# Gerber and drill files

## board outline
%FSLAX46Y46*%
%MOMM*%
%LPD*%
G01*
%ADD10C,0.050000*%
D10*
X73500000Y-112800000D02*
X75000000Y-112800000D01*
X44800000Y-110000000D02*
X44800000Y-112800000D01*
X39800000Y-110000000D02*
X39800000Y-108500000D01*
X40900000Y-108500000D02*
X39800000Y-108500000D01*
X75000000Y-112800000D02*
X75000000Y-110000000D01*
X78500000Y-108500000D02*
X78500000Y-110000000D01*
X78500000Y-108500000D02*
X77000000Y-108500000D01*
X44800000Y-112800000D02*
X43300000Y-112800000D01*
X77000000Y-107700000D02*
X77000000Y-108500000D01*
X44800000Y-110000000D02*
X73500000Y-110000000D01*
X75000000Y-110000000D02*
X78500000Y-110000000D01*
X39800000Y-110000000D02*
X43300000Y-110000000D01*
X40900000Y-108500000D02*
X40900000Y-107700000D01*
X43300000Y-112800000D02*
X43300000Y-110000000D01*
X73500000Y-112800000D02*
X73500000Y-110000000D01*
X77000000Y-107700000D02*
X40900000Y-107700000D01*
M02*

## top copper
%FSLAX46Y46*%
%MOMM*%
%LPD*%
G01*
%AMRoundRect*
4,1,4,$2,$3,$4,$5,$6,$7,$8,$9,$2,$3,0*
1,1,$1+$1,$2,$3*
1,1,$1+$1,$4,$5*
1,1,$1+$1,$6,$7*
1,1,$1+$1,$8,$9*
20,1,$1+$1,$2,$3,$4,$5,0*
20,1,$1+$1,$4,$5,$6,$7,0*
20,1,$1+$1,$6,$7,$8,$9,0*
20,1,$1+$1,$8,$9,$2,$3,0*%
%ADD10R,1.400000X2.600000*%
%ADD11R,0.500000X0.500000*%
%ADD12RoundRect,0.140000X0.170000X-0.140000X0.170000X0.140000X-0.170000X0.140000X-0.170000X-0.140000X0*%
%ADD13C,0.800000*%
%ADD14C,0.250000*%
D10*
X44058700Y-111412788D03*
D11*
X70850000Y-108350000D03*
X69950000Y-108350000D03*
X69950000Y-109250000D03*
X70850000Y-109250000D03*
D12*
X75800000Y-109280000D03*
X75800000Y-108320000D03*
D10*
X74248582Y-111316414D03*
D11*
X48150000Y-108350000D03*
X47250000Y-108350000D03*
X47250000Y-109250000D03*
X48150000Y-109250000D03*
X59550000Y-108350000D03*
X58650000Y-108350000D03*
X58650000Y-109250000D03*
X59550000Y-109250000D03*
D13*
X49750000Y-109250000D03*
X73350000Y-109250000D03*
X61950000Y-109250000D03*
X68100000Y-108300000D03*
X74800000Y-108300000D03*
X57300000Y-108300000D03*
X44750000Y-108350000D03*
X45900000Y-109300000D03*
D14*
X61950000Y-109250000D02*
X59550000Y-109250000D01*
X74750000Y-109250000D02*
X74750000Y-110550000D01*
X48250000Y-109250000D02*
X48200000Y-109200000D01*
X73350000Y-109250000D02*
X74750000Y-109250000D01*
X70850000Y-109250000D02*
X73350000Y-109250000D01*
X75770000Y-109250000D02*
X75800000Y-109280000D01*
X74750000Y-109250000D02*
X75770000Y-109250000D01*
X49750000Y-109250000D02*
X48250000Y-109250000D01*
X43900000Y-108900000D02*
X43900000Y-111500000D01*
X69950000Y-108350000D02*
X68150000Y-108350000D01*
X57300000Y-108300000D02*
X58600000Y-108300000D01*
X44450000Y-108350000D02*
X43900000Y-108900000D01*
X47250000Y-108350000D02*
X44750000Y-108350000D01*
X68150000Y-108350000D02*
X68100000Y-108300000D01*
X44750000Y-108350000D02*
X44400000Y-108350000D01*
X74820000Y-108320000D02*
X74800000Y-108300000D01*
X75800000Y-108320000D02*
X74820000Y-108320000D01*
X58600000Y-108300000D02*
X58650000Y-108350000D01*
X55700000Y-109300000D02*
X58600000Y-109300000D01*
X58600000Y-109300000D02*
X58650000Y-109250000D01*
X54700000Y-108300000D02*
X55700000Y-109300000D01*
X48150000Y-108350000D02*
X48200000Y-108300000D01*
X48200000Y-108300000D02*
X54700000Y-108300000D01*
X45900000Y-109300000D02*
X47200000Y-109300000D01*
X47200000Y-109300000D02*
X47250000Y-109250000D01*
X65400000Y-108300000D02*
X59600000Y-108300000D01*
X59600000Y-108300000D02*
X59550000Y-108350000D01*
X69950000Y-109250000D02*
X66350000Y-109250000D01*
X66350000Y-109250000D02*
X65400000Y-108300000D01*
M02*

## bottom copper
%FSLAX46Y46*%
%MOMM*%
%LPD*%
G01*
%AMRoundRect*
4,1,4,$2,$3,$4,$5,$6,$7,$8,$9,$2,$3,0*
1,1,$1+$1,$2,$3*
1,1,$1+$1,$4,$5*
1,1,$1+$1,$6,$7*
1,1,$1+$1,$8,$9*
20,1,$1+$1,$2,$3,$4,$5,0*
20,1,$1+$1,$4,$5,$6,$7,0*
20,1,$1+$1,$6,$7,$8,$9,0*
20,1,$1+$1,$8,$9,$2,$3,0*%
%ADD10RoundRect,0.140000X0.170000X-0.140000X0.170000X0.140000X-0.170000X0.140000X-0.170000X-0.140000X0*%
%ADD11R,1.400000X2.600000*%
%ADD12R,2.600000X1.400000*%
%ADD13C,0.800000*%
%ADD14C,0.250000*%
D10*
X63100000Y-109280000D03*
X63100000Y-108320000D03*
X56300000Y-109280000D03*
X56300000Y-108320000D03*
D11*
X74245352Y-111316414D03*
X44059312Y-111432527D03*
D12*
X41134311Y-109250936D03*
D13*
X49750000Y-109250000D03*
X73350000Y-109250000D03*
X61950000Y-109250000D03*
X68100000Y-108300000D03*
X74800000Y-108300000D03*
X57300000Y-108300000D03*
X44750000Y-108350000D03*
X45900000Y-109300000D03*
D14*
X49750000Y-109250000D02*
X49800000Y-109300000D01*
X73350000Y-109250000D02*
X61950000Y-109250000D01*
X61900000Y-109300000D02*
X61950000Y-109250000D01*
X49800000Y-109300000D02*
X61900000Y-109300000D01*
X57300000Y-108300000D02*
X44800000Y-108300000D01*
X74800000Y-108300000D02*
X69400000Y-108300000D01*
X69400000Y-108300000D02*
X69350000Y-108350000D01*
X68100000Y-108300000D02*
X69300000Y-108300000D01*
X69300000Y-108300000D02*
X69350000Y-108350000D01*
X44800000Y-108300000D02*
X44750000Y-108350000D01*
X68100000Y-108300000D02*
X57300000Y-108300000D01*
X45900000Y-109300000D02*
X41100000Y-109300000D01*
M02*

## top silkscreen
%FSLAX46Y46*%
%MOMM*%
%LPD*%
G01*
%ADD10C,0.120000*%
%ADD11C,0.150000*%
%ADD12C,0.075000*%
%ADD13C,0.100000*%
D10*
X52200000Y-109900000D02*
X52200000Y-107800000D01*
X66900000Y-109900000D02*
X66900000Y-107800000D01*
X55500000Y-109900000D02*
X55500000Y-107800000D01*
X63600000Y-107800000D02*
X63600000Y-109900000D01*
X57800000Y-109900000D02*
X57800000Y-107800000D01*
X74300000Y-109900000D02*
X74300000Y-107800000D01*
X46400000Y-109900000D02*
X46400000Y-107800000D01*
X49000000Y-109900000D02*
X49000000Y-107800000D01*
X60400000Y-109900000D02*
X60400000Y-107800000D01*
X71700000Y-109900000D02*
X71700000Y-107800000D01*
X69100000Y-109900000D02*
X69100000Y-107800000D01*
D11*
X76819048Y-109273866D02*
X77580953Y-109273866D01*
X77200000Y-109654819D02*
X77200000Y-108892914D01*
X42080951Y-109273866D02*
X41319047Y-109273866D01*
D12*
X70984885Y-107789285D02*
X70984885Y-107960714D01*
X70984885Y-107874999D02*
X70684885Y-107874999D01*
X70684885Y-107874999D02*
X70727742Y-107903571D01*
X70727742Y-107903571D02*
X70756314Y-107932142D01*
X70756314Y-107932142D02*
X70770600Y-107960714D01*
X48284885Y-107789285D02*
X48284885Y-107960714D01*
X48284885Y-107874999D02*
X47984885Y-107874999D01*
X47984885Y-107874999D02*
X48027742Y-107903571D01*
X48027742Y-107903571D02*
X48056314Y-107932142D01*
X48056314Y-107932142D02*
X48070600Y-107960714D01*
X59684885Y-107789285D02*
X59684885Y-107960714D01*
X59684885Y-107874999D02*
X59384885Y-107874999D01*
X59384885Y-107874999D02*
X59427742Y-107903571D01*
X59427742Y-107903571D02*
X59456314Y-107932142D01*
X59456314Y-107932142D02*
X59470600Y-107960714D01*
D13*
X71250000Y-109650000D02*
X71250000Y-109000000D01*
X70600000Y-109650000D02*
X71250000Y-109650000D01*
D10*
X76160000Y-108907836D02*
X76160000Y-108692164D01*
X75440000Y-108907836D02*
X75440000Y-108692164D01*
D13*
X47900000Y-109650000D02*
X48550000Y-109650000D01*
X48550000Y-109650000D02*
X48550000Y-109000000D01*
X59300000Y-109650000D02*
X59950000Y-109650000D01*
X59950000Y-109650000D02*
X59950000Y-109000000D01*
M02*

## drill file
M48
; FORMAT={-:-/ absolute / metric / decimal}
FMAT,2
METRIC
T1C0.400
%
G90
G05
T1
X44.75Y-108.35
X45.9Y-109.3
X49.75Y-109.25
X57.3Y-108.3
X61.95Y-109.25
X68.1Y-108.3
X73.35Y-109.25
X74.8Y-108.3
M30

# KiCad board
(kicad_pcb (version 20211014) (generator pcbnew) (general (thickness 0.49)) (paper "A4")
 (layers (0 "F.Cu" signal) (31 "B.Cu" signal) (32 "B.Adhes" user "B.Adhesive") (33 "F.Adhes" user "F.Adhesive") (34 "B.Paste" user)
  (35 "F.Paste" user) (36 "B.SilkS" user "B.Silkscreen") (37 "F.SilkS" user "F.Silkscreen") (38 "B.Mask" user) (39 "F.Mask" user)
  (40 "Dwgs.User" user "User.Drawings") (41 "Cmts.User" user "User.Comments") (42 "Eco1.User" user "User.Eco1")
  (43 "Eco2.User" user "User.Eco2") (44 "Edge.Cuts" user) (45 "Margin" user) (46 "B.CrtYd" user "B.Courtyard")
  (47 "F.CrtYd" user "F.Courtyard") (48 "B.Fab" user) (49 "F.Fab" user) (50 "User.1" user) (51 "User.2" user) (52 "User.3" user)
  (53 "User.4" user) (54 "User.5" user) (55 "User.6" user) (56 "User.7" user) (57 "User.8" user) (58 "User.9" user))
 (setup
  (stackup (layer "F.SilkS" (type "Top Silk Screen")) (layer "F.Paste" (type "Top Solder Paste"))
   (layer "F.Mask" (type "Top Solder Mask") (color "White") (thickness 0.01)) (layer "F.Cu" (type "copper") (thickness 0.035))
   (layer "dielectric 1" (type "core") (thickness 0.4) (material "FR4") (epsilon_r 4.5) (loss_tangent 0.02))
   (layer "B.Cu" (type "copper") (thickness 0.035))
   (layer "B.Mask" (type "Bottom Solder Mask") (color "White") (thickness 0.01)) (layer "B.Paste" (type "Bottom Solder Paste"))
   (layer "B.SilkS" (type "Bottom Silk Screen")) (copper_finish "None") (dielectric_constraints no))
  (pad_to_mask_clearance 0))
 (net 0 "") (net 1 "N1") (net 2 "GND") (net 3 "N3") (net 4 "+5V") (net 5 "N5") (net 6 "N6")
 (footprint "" (layer "F.Cu") (at 44.0587 111.412788)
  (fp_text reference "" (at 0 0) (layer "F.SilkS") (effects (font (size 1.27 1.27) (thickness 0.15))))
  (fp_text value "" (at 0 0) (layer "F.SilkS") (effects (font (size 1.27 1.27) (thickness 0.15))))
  (pad "" smd rect (at 0 0) (size 1.4 2.6) (layers "F.Cu" "F.Paste" "F.Mask")))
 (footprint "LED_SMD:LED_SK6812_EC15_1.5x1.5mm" (layer "F.Cu") (at 70.4 108.8 -90)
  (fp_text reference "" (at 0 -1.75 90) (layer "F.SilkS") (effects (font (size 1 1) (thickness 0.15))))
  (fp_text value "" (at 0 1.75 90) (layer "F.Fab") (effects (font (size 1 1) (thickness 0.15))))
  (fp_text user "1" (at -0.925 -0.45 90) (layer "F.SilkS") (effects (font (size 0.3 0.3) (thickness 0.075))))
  (fp_line (start 0.85 -0.85) (end 0.2 -0.85) (layer "F.SilkS") (width 0.1))
  (fp_line (start 0.85 -0.2) (end 0.85 -0.85) (layer "F.SilkS") (width 0.1))
  (pad "1" smd rect (at -0.45 -0.45 270) (size 0.5 0.5) (layers "F.Cu" "F.Paste" "F.Mask") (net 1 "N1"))
  (pad "2" smd rect (at -0.45 0.45 270) (size 0.5 0.5) (layers "F.Cu" "F.Paste" "F.Mask") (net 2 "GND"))
  (pad "3" smd rect (at 0.45 0.45 270) (size 0.5 0.5) (layers "F.Cu" "F.Paste" "F.Mask") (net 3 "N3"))
  (pad "4" smd rect (at 0.45 -0.45 270) (size 0.5 0.5) (layers "F.Cu" "F.Paste" "F.Mask") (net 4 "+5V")))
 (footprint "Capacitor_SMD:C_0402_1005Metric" (layer "F.Cu") (at 75.8 108.8 90)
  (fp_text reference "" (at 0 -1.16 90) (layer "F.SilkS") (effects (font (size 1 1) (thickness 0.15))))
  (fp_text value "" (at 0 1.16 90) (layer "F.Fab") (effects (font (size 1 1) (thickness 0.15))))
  (fp_line (start -0.107836 0.36) (end 0.107836 0.36) (layer "F.SilkS") (width 0.12))
  (fp_line (start -0.107836 -0.36) (end 0.107836 -0.36) (layer "F.SilkS") (width 0.12))
  (pad "1" smd roundrect (at -0.48 0 90) (size 0.56 0.62) (layers "F.Cu" "F.Paste" "F.Mask") (roundrect_rratio 0.25) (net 4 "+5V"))
  (pad "2" smd roundrect (at 0.48 0 90) (size 0.56 0.62) (layers "F.Cu" "F.Paste" "F.Mask") (roundrect_rratio 0.25) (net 2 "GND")))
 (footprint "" (layer "F.Cu") (at 74.248582 111.316414)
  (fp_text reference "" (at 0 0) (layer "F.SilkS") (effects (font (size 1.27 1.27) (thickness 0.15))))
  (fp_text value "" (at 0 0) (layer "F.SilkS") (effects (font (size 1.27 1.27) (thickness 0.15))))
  (pad "" smd rect (at 0 0) (size 1.4 2.6) (layers "F.Cu" "F.Paste" "F.Mask")))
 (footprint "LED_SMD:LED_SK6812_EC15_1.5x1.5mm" (layer "F.Cu") (at 47.7 108.8 -90)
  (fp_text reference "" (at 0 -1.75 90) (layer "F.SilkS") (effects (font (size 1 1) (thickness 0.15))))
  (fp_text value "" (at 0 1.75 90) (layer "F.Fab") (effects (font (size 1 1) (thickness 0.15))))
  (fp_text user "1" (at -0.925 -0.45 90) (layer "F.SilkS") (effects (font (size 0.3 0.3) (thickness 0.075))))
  (fp_line (start 0.85 -0.2) (end 0.85 -0.85) (layer "F.SilkS") (width 0.1))
  (fp_line (start 0.85 -0.85) (end 0.2 -0.85) (layer "F.SilkS") (width 0.1))
  (pad "1" smd rect (at -0.45 -0.45 270) (size 0.5 0.5) (layers "F.Cu" "F.Paste" "F.Mask") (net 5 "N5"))
  (pad "2" smd rect (at -0.45 0.45 270) (size 0.5 0.5) (layers "F.Cu" "F.Paste" "F.Mask") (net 2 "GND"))
  (pad "3" smd rect (at 0.45 0.45 270) (size 0.5 0.5) (layers "F.Cu" "F.Paste" "F.Mask") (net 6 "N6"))
  (pad "4" smd rect (at 0.45 -0.45 270) (size 0.5 0.5) (layers "F.Cu" "F.Paste" "F.Mask") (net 4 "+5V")))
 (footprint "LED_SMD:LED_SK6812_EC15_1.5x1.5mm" (layer "F.Cu") (at 59.1 108.8 -90)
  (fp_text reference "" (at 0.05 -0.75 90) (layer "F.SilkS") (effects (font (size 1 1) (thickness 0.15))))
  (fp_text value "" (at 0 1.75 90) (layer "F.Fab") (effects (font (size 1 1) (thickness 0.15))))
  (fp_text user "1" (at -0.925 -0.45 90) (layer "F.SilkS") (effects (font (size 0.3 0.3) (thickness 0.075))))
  (fp_line (start 0.85 -0.2) (end 0.85 -0.85) (layer "F.SilkS") (width 0.1))
  (fp_line (start 0.85 -0.85) (end 0.2 -0.85) (layer "F.SilkS") (width 0.1))
  (pad "1" smd rect (at -0.45 -0.45 270) (size 0.5 0.5) (layers "F.Cu" "F.Paste" "F.Mask") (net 3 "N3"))
  (pad "2" smd rect (at -0.45 0.45 270) (size 0.5 0.5) (layers "F.Cu" "F.Paste" "F.Mask") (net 2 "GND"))
  (pad "3" smd rect (at 0.45 0.45 270) (size 0.5 0.5) (layers "F.Cu" "F.Paste" "F.Mask") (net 5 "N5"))
  (pad "4" smd rect (at 0.45 -0.45 270) (size 0.5 0.5) (layers "F.Cu" "F.Paste" "F.Mask") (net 4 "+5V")))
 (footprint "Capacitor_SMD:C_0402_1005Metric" (layer "B.Cu") (at 63.1 108.8 90)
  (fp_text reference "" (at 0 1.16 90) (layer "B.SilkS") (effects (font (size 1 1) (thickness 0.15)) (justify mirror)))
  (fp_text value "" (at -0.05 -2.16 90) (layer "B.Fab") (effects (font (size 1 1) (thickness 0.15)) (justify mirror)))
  (pad "1" smd roundrect (at -0.48 0 90) (size 0.56 0.62) (layers "B.Cu" "B.Paste" "B.Mask") (roundrect_rratio 0.25))
  (pad "2" smd roundrect (at 0.48 0 90) (size 0.56 0.62) (layers "B.Cu" "B.Paste" "B.Mask") (roundrect_rratio 0.25)))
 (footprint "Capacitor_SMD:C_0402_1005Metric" (layer "B.Cu") (at 56.3 108.8 90)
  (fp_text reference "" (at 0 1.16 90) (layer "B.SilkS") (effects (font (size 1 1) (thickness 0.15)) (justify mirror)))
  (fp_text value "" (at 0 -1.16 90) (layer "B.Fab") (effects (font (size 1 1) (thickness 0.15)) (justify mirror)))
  (pad "1" smd roundrect (at -0.48 0 90) (size 0.56 0.62) (layers "B.Cu" "B.Paste" "B.Mask") (roundrect_rratio 0.25))
  (pad "2" smd roundrect (at 0.48 0 90) (size 0.56 0.62) (layers "B.Cu" "B.Paste" "B.Mask") (roundrect_rratio 0.25)))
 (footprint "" (layer "B.Cu") (at 74.245352 111.316414 180)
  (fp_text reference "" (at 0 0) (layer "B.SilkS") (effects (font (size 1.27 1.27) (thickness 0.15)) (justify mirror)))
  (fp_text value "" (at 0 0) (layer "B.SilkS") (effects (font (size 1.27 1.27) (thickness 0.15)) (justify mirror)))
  (pad "" smd rect (at 0 0 180) (size 1.4 2.6) (layers "B.Cu" "B.Paste" "B.Mask")))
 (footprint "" (layer "B.Cu") (at 44.059312 111.432527 180)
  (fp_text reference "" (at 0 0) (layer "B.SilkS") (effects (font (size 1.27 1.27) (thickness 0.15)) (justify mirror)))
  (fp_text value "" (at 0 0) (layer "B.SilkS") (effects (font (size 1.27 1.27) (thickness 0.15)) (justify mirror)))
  (pad "" smd rect (at 0 0 180) (size 1.4 2.6) (layers "B.Cu" "B.Paste" "B.Mask")))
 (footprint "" (layer "B.Cu") (at 41.134311 109.250936 90)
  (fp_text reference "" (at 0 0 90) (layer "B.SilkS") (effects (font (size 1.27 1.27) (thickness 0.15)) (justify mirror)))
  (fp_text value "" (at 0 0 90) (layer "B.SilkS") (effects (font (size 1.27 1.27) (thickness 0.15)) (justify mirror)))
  (pad "" smd rect (at 0 0 90) (size 1.4 2.6) (layers "B.Cu" "B.Paste" "B.Mask")))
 (gr_line (start 52.2 109.9) (end 52.2 107.8) (layer "F.SilkS") (width 0.12))
 (gr_line (start 66.9 109.9) (end 66.9 107.8) (layer "F.SilkS") (width 0.12))
 (gr_line (start 55.5 109.9) (end 55.5 107.8) (layer "F.SilkS") (width 0.12))
 (gr_line (start 63.6 107.8) (end 63.6 109.9) (layer "F.SilkS") (width 0.12))
 (gr_line (start 57.8 109.9) (end 57.8 107.8) (layer "F.SilkS") (width 0.12))
 (gr_line (start 74.3 109.9) (end 74.3 107.8) (layer "F.SilkS") (width 0.12))
 (gr_line (start 46.4 109.9) (end 46.4 107.8) (layer "F.SilkS") (width 0.12))
 (gr_line (start 49 109.9) (end 49 107.8) (layer "F.SilkS") (width 0.12))
 (gr_line (start 60.4 109.9) (end 60.4 107.8) (layer "F.SilkS") (width 0.12))
 (gr_line (start 71.7 109.9) (end 71.7 107.8) (layer "F.SilkS") (width 0.12))
 (gr_line (start 69.1 109.9) (end 69.1 107.8) (layer "F.SilkS") (width 0.12))
 (gr_line (start 73.5 112.8) (end 75 112.8) (layer "Edge.Cuts") (width 0.05))
 (gr_line (start 44.8 110) (end 44.8 112.8) (layer "Edge.Cuts") (width 0.05))
 (gr_line (start 39.8 110) (end 39.8 108.5) (layer "Edge.Cuts") (width 0.05))
 (gr_line (start 40.9 108.5) (end 39.8 108.5) (layer "Edge.Cuts") (width 0.05))
 (gr_line (start 75 112.8) (end 75 110) (layer "Edge.Cuts") (width 0.05))
 (gr_line (start 78.5 108.5) (end 78.5 110) (layer "Edge.Cuts") (width 0.05))
 (gr_line (start 78.5 108.5) (end 77 108.5) (layer "Edge.Cuts") (width 0.05))
 (gr_line (start 44.8 112.8) (end 43.3 112.8) (layer "Edge.Cuts") (width 0.05))
 (gr_line (start 77 107.7) (end 77 108.5) (layer "Edge.Cuts") (width 0.05))
 (gr_line (start 44.8 110) (end 73.5 110) (layer "Edge.Cuts") (width 0.05))
 (gr_line (start 75 110) (end 78.5 110) (layer "Edge.Cuts") (width 0.05))
 (gr_line (start 39.8 110) (end 43.3 110) (layer "Edge.Cuts") (width 0.05))
 (gr_line (start 40.9 108.5) (end 40.9 107.7) (layer "Edge.Cuts") (width 0.05))
 (gr_line (start 43.3 112.8) (end 43.3 110) (layer "Edge.Cuts") (width 0.05))
 (gr_line (start 73.5 112.8) (end 73.5 110) (layer "Edge.Cuts") (width 0.05))
 (gr_line (start 77 107.7) (end 40.9 107.7) (layer "Edge.Cuts") (width 0.05))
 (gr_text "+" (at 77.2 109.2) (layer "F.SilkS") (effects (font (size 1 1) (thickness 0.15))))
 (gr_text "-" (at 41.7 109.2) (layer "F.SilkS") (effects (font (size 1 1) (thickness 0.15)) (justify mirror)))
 (segment (start 61.95 109.25) (end 59.55 109.25) (width 0.25) (layer "F.Cu") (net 4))
 (segment (start 74.75 109.25) (end 74.75 110.55) (width 0.25) (layer "F.Cu") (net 4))
 (segment (start 48.25 109.25) (end 48.2 109.2) (width 0.25) (layer "F.Cu") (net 4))
 (segment (start 73.35 109.25) (end 74.75 109.25) (width 0.25) (layer "F.Cu") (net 4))
 (segment (start 70.85 109.25) (end 73.35 109.25) (width 0.25) (layer "F.Cu") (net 4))
 (segment (start 75.77 109.25) (end 75.8 109.28) (width 0.25) (layer "F.Cu") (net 4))
 (segment (start 74.75 109.25) (end 75.77 109.25) (width 0.25) (layer "F.Cu") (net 4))
 (segment (start 49.75 109.25) (end 48.25 109.25) (width 0.25) (layer "F.Cu") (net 4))
 (via (at 49.75 109.25) (size 0.8) (drill 0.4) (layers "F.Cu" "B.Cu") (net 4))
 (via (at 73.35 109.25) (size 0.8) (drill 0.4) (layers "F.Cu" "B.Cu") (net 4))
 (via (at 61.95 109.25) (size 0.8) (drill 0.4) (layers "F.Cu" "B.Cu") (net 4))
 (segment (start 49.75 109.25) (end 49.8 109.3) (width 0.25) (layer "B.Cu") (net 4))
 (segment (start 73.35 109.25) (end 61.95 109.25) (width 0.25) (layer "B.Cu") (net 4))
 (segment (start 61.9 109.3) (end 61.95 109.25) (width 0.25) (layer "B.Cu") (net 4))
 (segment (start 49.8 109.3) (end 61.9 109.3) (width 0.25) (layer "B.Cu") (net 4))
 (segment (start 43.9 108.9) (end 43.9 111.5) (width 0.25) (layer "F.Cu") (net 2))
 (segment (start 69.95 108.35) (end 68.15 108.35) (width 0.25) (layer "F.Cu") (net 2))
 (segment (start 57.3 108.3) (end 58.6 108.3) (width 0.25) (layer "F.Cu") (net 2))
 (segment (start 44.45 108.35) (end 43.9 108.9) (width 0.25) (layer "F.Cu") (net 2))
 (segment (start 47.25 108.35) (end 44.75 108.35) (width 0.25) (layer "F.Cu") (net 2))
 (segment (start 68.15 108.35) (end 68.1 108.3) (width 0.25) (layer "F.Cu") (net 2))
 (segment (start 44.75 108.35) (end 44.4 108.35) (width 0.25) (layer "F.Cu") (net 2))
 (segment (start 74.82 108.32) (end 74.8 108.3) (width 0.25) (layer "F.Cu") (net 2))
 (segment (start 75.8 108.32) (end 74.82 108.32) (width 0.25) (layer "F.Cu") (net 2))
 (segment (start 58.6 108.3) (end 58.65 108.35) (width 0.25) (layer "F.Cu") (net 2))
 (via (at 68.1 108.3) (size 0.8) (drill 0.4) (layers "F.Cu" "B.Cu") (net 2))
 (via (at 74.8 108.3) (size 0.8) (drill 0.4) (layers "F.Cu" "B.Cu") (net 2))
 (via (at 57.3 108.3) (size 0.8) (drill 0.4) (layers "F.Cu" "B.Cu") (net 2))
 (via (at 44.75 108.35) (size 0.8) (drill 0.4) (layers "F.Cu" "B.Cu") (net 2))
 (segment (start 57.3 108.3) (end 44.8 108.3) (width 0.25) (layer "B.Cu") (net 2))
 (segment (start 74.8 108.3) (end 69.4 108.3) (width 0.25) (layer "B.Cu") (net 2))
 (segment (start 69.4 108.3) (end 69.35 108.35) (width 0.25) (layer "B.Cu") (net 2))
 (segment (start 68.1 108.3) (end 69.3 108.3) (width 0.25) (layer "B.Cu") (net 2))
 (segment (start 69.3 108.3) (end 69.35 108.35) (width 0.25) (layer "B.Cu") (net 2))
 (segment (start 44.8 108.3) (end 44.75 108.35) (width 0.25) (layer "B.Cu") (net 2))
 (segment (start 68.1 108.3) (end 57.3 108.3) (width 0.25) (layer "B.Cu") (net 2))
 (segment (start 55.7 109.3) (end 58.6 109.3) (width 0.25) (layer "F.Cu") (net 5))
 (segment (start 58.6 109.3) (end 58.65 109.25) (width 0.25) (layer "F.Cu") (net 5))
 (segment (start 54.7 108.3) (end 55.7 109.3) (width 0.25) (layer "F.Cu") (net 5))
 (segment (start 48.15 108.35) (end 48.2 108.3) (width 0.25) (layer "F.Cu") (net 5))
 (segment (start 48.2 108.3) (end 54.7 108.3) (width 0.25) (layer "F.Cu") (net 5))
 (segment (start 45.9 109.3) (end 47.2 109.3) (width 0.25) (layer "F.Cu") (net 6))
 (segment (start 47.2 109.3) (end 47.25 109.25) (width 0.25) (layer "F.Cu") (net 6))
 (via (at 45.9 109.3) (size 0.8) (drill 0.4) (layers "F.Cu" "B.Cu") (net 6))
 (segment (start 45.9 109.3) (end 41.1 109.3) (width 0.25) (layer "B.Cu") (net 6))
 (segment (start 65.4 108.3) (end 59.6 108.3) (width 0.25) (layer "F.Cu") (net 3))
 (segment (start 59.6 108.3) (end 59.55 108.35) (width 0.25) (layer "F.Cu") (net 3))
 (segment (start 69.95 109.25) (end 66.35 109.25) (width 0.25) (layer "F.Cu") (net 3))
 (segment (start 66.35 109.25) (end 65.4 108.3) (width 0.25) (layer "F.Cu") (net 3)))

